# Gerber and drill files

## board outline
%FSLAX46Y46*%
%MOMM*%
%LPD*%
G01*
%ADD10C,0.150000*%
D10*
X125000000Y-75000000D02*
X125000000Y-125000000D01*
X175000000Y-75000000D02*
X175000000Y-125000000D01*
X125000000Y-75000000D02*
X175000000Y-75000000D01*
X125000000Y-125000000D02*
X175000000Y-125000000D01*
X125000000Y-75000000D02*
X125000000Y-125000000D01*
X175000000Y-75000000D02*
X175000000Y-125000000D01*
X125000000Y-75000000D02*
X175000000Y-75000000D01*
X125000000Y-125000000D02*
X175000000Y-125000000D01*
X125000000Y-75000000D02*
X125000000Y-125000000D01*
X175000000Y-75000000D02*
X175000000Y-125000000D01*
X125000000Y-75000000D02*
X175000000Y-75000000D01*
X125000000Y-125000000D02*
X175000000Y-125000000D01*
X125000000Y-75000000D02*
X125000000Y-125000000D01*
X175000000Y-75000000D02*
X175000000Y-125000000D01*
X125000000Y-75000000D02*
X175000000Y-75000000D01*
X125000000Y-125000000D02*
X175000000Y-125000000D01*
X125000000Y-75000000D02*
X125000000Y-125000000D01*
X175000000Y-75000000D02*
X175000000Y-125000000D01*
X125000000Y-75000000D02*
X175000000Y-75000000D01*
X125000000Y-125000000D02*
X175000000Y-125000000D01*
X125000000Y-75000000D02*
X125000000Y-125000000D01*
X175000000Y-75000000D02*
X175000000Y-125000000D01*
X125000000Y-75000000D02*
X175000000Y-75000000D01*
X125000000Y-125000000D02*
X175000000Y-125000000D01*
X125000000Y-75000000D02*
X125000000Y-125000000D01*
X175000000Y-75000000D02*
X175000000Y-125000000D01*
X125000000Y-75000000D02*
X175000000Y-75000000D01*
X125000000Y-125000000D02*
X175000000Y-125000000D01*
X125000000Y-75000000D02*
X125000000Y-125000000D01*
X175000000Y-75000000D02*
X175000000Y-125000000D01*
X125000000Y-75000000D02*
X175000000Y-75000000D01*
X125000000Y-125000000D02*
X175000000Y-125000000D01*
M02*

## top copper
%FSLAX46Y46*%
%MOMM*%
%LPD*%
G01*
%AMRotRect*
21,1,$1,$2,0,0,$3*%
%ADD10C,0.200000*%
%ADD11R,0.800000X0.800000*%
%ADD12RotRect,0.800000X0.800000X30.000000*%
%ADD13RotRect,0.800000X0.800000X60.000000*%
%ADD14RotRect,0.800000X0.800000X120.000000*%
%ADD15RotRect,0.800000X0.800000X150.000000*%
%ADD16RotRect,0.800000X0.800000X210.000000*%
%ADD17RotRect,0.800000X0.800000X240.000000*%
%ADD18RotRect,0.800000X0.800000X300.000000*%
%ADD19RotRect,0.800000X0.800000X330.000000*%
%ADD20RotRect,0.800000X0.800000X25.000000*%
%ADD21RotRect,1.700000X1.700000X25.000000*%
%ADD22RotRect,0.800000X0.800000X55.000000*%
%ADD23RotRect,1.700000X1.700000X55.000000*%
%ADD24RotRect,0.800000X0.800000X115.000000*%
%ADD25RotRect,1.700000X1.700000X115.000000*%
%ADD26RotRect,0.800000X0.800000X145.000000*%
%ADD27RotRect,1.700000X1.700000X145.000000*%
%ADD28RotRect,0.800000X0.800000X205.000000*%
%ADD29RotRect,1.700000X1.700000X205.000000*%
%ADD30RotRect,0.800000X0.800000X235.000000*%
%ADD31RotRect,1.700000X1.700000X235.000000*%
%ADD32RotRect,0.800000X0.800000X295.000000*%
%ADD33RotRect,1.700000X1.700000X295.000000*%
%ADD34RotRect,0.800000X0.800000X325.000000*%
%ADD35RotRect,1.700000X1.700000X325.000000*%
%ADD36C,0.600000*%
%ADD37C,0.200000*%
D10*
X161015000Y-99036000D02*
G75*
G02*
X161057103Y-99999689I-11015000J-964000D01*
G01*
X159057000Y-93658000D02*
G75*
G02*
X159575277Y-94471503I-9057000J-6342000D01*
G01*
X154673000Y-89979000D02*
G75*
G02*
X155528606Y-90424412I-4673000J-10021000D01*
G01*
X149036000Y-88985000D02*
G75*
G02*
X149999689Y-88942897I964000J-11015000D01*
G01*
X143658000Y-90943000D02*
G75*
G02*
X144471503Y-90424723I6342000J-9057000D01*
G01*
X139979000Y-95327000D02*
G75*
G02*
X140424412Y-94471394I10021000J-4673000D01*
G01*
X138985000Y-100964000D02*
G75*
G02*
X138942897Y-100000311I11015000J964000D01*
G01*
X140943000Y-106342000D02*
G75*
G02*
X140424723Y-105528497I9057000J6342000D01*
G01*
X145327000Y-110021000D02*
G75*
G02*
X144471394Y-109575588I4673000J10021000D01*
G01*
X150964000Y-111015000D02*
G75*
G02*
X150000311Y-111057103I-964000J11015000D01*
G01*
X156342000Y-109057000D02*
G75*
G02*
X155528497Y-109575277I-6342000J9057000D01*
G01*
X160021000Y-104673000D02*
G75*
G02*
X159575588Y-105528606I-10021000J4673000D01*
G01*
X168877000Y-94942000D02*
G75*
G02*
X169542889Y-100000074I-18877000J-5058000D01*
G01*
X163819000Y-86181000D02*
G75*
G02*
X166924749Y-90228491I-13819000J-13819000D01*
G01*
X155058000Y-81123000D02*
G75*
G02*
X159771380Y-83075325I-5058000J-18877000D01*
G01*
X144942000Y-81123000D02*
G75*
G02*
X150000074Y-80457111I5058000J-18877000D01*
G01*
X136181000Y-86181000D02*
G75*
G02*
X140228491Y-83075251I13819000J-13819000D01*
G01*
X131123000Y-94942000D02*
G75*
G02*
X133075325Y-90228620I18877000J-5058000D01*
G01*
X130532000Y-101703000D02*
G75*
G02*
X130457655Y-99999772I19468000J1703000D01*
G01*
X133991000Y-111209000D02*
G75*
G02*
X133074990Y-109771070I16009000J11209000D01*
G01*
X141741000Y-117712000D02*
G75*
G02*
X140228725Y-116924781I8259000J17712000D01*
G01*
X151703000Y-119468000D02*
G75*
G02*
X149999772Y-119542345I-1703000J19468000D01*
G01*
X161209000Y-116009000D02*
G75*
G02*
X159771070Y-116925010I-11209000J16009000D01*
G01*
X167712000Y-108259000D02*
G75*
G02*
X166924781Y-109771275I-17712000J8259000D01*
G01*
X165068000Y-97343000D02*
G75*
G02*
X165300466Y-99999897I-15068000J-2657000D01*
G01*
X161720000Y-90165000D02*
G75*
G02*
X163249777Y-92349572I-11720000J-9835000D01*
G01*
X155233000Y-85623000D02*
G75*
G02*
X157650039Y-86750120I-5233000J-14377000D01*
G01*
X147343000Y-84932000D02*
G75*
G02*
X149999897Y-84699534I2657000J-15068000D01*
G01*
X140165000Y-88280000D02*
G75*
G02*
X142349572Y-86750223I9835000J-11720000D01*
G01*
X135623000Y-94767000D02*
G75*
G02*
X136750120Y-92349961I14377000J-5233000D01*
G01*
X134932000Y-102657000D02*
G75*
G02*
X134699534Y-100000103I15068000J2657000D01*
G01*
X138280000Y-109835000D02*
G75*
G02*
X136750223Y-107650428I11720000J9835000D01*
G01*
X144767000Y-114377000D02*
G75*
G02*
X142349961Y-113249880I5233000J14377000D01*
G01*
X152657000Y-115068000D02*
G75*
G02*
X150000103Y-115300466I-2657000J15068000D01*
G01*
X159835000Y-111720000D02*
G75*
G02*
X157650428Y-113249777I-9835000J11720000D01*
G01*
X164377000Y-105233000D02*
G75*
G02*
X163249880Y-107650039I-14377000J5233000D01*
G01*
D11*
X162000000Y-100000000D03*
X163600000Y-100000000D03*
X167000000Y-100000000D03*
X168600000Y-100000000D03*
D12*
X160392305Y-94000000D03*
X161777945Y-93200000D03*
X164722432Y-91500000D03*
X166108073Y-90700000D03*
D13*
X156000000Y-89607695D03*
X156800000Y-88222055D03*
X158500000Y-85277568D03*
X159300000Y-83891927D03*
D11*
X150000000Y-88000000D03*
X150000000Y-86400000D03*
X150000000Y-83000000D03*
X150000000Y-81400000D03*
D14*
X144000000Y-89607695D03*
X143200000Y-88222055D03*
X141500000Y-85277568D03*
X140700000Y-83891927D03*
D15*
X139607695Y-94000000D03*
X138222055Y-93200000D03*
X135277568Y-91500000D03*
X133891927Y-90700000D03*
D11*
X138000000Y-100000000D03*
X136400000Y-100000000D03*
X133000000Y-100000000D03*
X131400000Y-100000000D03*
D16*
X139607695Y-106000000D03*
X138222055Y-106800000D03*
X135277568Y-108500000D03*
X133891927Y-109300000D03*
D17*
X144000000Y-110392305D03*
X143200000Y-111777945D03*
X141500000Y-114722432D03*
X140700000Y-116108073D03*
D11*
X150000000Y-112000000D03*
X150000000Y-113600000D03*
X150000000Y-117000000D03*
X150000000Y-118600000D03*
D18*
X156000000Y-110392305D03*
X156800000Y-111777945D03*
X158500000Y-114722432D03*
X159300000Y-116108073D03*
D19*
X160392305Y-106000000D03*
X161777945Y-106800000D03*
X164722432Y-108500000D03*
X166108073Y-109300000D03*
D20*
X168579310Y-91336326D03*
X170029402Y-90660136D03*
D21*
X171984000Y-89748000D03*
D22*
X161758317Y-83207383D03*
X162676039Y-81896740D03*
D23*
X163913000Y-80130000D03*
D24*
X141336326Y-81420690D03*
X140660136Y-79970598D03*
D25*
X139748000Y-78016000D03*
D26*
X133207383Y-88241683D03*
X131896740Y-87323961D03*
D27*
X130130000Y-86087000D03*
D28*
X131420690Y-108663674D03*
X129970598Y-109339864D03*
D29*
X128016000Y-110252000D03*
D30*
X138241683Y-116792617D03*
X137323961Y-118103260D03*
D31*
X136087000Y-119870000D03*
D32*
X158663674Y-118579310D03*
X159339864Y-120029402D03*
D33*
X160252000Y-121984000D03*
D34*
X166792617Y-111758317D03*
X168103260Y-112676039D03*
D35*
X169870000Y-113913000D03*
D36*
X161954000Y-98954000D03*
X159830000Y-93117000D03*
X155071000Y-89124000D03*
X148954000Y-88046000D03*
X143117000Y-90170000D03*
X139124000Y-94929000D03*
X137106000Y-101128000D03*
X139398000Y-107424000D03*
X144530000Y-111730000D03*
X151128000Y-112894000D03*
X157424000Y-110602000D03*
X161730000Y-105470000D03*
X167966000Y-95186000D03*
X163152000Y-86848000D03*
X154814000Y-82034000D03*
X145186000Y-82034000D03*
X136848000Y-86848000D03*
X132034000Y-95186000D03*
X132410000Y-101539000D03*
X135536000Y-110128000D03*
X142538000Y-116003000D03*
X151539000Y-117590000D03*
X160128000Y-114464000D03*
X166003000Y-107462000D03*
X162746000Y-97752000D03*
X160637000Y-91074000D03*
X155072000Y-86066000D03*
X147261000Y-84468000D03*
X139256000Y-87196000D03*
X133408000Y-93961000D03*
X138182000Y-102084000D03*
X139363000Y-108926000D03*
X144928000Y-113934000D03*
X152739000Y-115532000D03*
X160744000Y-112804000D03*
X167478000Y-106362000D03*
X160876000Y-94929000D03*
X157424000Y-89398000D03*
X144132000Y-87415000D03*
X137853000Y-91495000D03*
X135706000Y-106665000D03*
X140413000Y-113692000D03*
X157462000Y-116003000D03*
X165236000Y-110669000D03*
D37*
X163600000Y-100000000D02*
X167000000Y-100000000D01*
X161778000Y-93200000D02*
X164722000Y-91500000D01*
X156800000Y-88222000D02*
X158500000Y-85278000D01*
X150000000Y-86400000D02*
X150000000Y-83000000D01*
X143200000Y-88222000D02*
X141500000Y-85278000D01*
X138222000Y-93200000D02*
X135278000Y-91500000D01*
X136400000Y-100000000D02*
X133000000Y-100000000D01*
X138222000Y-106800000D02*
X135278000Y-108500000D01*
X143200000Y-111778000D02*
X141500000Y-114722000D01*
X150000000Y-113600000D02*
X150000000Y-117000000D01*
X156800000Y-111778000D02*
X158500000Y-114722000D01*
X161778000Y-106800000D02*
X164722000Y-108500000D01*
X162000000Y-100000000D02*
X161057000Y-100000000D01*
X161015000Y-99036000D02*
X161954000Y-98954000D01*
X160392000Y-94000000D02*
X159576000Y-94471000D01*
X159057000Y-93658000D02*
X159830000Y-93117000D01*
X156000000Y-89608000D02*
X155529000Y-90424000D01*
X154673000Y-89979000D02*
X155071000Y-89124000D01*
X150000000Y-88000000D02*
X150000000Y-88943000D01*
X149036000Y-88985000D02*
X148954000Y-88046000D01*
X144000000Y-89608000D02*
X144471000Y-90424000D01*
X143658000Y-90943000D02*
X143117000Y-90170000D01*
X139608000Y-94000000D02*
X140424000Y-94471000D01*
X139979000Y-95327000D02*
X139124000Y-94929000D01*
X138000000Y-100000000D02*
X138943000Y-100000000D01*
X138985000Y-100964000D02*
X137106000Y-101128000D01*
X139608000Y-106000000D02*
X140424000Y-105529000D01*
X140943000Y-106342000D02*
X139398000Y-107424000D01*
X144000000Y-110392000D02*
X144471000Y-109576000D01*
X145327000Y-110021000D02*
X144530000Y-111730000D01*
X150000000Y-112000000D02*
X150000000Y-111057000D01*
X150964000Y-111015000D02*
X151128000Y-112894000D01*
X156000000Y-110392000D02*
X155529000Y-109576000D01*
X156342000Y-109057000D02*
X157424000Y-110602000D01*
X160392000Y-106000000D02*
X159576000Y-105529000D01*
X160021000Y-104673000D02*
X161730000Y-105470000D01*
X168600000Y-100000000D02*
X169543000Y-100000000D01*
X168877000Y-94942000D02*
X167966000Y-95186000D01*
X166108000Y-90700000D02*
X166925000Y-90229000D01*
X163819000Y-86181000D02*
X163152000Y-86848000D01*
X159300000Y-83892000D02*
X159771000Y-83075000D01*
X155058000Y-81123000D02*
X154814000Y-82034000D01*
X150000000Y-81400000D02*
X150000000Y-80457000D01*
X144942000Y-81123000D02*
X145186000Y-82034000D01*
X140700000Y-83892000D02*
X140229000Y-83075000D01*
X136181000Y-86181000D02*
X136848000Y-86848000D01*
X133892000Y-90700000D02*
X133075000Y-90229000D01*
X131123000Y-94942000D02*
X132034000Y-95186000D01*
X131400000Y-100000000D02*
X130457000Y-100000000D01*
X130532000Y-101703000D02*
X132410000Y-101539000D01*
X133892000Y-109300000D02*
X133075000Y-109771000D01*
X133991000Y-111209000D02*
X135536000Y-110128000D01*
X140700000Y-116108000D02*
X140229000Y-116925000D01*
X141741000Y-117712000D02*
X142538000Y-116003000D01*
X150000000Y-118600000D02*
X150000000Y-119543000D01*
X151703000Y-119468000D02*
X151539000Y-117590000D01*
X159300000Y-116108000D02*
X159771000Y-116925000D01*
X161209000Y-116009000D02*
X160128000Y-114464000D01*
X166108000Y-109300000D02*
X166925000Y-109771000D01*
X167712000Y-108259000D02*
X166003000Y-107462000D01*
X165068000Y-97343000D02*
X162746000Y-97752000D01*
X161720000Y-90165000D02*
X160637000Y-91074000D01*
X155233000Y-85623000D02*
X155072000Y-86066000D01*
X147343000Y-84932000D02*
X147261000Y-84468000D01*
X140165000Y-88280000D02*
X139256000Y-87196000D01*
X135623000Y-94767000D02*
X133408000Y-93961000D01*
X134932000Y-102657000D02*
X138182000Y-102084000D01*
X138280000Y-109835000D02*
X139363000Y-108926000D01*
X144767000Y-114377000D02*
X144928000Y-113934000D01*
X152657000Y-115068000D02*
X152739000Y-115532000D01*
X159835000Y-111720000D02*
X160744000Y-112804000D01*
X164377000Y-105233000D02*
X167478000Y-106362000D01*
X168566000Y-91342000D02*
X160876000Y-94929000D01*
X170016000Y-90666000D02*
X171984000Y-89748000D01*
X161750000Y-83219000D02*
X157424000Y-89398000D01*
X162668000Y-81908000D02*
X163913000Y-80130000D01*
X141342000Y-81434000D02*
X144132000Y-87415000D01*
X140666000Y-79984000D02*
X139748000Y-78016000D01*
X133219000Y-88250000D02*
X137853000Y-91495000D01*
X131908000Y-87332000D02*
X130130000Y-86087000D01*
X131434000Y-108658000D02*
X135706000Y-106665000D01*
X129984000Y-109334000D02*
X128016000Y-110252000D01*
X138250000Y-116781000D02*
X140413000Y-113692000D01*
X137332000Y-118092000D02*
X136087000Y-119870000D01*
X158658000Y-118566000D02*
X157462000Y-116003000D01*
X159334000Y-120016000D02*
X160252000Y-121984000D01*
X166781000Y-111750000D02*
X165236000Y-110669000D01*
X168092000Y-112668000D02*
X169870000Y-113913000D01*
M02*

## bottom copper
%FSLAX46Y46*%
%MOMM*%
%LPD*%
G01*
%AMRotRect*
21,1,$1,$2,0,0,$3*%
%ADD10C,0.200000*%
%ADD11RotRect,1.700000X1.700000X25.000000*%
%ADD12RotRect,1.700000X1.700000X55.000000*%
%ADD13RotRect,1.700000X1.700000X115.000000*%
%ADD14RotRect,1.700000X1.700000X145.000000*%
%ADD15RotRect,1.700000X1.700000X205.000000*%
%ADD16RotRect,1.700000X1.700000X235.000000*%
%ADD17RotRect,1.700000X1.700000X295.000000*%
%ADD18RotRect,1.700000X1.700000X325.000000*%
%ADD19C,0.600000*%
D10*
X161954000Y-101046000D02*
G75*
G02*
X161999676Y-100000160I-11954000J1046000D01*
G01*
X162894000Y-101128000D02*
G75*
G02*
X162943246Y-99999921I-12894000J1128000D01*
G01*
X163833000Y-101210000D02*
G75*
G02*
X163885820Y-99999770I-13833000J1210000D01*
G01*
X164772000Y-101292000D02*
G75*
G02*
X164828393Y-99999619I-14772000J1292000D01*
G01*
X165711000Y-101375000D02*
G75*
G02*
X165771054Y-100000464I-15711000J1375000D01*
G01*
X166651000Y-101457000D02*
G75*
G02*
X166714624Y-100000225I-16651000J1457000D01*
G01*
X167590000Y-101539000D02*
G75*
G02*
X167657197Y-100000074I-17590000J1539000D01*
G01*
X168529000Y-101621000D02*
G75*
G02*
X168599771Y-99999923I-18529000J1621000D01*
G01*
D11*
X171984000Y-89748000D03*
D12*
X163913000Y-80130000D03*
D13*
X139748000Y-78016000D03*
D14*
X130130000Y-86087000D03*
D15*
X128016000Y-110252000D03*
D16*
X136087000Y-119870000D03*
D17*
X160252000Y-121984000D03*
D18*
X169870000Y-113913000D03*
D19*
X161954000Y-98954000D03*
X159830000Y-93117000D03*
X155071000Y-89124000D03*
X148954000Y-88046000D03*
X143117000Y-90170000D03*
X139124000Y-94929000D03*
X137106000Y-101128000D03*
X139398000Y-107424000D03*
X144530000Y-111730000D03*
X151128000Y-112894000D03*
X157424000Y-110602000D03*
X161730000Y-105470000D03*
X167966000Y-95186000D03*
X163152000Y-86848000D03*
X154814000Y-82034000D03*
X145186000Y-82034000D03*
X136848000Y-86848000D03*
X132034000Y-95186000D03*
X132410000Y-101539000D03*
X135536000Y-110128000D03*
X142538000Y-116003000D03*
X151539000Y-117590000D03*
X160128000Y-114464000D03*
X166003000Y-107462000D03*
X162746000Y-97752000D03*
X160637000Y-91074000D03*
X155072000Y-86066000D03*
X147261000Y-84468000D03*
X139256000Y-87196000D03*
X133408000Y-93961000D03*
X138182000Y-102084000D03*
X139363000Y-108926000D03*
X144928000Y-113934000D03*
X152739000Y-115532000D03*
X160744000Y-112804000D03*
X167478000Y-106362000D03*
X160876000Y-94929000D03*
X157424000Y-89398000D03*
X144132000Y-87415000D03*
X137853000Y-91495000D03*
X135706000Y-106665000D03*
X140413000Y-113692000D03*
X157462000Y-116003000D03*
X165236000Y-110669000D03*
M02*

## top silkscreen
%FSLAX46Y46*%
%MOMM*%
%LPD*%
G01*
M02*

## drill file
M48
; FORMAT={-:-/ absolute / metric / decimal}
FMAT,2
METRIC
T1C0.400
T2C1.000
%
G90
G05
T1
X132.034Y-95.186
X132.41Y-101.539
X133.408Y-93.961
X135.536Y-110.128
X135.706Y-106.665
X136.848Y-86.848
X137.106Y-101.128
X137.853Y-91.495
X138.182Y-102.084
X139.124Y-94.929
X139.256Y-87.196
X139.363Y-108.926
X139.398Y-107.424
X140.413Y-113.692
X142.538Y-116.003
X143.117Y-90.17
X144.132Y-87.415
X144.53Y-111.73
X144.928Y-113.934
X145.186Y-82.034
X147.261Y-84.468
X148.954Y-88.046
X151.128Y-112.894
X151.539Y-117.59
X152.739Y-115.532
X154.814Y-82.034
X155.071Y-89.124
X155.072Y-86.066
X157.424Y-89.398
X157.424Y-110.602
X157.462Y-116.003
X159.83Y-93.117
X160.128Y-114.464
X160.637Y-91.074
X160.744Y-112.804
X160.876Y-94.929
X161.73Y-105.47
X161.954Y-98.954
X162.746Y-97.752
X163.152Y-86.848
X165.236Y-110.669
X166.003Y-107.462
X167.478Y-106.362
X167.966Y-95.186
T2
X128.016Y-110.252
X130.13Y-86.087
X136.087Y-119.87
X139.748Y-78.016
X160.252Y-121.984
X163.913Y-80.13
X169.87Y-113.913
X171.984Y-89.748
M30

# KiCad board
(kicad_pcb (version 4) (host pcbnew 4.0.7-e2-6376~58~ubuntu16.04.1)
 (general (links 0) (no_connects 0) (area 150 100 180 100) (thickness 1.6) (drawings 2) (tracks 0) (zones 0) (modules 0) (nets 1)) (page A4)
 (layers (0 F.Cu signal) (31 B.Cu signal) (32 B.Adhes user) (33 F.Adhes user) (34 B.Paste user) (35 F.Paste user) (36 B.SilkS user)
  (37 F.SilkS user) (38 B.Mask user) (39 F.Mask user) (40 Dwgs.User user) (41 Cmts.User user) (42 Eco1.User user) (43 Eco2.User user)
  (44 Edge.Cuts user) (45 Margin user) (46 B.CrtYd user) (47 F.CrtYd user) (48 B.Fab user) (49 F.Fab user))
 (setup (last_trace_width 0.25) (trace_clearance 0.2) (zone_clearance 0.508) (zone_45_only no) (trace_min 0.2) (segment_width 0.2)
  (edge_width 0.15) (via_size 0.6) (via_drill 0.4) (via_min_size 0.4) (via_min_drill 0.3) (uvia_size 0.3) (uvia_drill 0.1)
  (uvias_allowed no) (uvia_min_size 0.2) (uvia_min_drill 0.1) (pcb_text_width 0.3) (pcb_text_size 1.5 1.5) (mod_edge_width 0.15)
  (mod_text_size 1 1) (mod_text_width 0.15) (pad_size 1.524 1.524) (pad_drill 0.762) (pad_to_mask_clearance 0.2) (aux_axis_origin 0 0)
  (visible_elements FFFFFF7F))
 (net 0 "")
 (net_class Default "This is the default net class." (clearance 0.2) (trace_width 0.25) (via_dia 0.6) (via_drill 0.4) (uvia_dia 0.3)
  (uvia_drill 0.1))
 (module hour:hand (layer F.Cu) (at 150 100 0.0)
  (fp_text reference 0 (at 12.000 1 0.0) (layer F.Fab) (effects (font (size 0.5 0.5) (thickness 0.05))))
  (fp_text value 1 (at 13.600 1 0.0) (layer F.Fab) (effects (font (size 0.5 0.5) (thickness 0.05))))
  (pad 1 smd rect (at 12.0 0 0.0) (size 0.8 0.8) (layers F.Cu F.Paste F.Mask))
  (pad 2 smd rect (at 13.6 0 0.0) (size 0.8 0.8) (layers F.Cu F.Paste F.Mask)))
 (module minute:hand (layer F.Cu) (at 150 100 0.0)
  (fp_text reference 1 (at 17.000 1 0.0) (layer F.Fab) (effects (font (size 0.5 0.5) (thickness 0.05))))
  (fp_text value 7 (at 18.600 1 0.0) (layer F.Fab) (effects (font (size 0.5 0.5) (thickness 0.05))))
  (pad 1 smd rect (at 17.0 0 0.0) (size 0.8 0.8) (layers F.Cu F.Paste F.Mask))
  (pad 2 smd rect (at 18.6 0 0.0) (size 0.8 0.8) (layers F.Cu F.Paste F.Mask)))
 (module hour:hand (layer F.Cu) (at 150 100 30.0)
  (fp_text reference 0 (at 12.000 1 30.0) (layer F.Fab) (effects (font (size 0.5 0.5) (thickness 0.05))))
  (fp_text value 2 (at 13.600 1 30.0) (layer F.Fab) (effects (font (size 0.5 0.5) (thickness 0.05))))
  (pad 1 smd rect (at 12.0 0 30.0) (size 0.8 0.8) (layers F.Cu F.Paste F.Mask))
  (pad 2 smd rect (at 13.6 0 30.0) (size 0.8 0.8) (layers F.Cu F.Paste F.Mask)))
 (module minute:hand (layer F.Cu) (at 150 100 30.0)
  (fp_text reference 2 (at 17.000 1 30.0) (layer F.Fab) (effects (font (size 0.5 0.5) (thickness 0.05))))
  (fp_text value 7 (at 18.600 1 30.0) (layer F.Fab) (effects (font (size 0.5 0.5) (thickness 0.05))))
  (pad 1 smd rect (at 17.0 0 30.0) (size 0.8 0.8) (layers F.Cu F.Paste F.Mask))
  (pad 2 smd rect (at 18.6 0 30.0) (size 0.8 0.8) (layers F.Cu F.Paste F.Mask)))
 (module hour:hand (layer F.Cu) (at 150 100 60.0)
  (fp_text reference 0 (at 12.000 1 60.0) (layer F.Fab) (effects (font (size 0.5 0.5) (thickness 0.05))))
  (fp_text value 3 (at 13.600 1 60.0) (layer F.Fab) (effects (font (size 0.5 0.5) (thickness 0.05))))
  (pad 1 smd rect (at 12.0 0 60.0) (size 0.8 0.8) (layers F.Cu F.Paste F.Mask))
  (pad 2 smd rect (at 13.6 0 60.0) (size 0.8 0.8) (layers F.Cu F.Paste F.Mask)))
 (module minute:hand (layer F.Cu) (at 150 100 60.0)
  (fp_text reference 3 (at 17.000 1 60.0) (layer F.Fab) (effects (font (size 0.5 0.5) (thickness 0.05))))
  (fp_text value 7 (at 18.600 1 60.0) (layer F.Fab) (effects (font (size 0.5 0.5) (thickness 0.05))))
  (pad 1 smd rect (at 17.0 0 60.0) (size 0.8 0.8) (layers F.Cu F.Paste F.Mask))
  (pad 2 smd rect (at 18.6 0 60.0) (size 0.8 0.8) (layers F.Cu F.Paste F.Mask)))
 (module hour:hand (layer F.Cu) (at 150 100 90.0)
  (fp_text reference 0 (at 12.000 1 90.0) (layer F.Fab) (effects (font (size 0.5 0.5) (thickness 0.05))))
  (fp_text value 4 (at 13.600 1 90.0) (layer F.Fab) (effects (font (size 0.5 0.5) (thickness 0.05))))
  (pad 1 smd rect (at 12.0 0 90.0) (size 0.8 0.8) (layers F.Cu F.Paste F.Mask))
  (pad 2 smd rect (at 13.6 0 90.0) (size 0.8 0.8) (layers F.Cu F.Paste F.Mask)))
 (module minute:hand (layer F.Cu) (at 150 100 90.0)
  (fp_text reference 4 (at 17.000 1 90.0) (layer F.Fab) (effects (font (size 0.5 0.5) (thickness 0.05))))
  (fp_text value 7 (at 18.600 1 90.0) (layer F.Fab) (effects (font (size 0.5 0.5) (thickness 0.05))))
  (pad 1 smd rect (at 17.0 0 90.0) (size 0.8 0.8) (layers F.Cu F.Paste F.Mask))
  (pad 2 smd rect (at 18.6 0 90.0) (size 0.8 0.8) (layers F.Cu F.Paste F.Mask)))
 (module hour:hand (layer F.Cu) (at 150 100 120.0)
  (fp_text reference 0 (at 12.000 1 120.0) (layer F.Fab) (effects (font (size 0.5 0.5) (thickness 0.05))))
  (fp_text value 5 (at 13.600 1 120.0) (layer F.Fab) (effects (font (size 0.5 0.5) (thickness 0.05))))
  (pad 1 smd rect (at 12.0 0 120.0) (size 0.8 0.8) (layers F.Cu F.Paste F.Mask))
  (pad 2 smd rect (at 13.6 0 120.0) (size 0.8 0.8) (layers F.Cu F.Paste F.Mask)))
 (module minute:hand (layer F.Cu) (at 150 100 120.0)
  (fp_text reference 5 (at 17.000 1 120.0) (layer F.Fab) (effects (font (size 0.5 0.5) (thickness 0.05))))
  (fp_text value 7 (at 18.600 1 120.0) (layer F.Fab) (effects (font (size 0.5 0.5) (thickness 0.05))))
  (pad 1 smd rect (at 17.0 0 120.0) (size 0.8 0.8) (layers F.Cu F.Paste F.Mask))
  (pad 2 smd rect (at 18.6 0 120.0) (size 0.8 0.8) (layers F.Cu F.Paste F.Mask)))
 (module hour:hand (layer F.Cu) (at 150 100 150.0)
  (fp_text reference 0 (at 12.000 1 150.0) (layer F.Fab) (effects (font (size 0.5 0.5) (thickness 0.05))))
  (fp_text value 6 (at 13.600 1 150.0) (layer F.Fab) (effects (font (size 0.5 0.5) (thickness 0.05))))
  (pad 1 smd rect (at 12.0 0 150.0) (size 0.8 0.8) (layers F.Cu F.Paste F.Mask))
  (pad 2 smd rect (at 13.6 0 150.0) (size 0.8 0.8) (layers F.Cu F.Paste F.Mask)))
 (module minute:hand (layer F.Cu) (at 150 100 150.0)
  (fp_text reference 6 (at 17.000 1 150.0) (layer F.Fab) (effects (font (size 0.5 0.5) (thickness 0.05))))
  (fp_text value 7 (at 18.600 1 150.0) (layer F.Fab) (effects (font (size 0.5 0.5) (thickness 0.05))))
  (pad 1 smd rect (at 17.0 0 150.0) (size 0.8 0.8) (layers F.Cu F.Paste F.Mask))
  (pad 2 smd rect (at 18.6 0 150.0) (size 0.8 0.8) (layers F.Cu F.Paste F.Mask)))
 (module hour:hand (layer F.Cu) (at 150 100 180.0)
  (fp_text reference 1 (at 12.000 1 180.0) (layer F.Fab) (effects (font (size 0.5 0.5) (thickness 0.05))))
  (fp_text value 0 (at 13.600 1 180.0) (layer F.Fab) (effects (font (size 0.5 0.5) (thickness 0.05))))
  (pad 1 smd rect (at 12.0 0 180.0) (size 0.8 0.8) (layers F.Cu F.Paste F.Mask))
  (pad 2 smd rect (at 13.6 0 180.0) (size 0.8 0.8) (layers F.Cu F.Paste F.Mask)))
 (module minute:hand (layer F.Cu) (at 150 100 180.0)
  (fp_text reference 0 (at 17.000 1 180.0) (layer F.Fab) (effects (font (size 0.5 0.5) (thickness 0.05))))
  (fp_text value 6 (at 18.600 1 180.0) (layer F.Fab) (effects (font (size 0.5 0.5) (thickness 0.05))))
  (pad 1 smd rect (at 17.0 0 180.0) (size 0.8 0.8) (layers F.Cu F.Paste F.Mask))
  (pad 2 smd rect (at 18.6 0 180.0) (size 0.8 0.8) (layers F.Cu F.Paste F.Mask)))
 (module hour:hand (layer F.Cu) (at 150 100 210.0)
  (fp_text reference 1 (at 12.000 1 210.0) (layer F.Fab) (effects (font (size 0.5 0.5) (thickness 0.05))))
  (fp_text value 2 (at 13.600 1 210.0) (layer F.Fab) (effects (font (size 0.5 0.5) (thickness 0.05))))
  (pad 1 smd rect (at 12.0 0 210.0) (size 0.8 0.8) (layers F.Cu F.Paste F.Mask))
  (pad 2 smd rect (at 13.6 0 210.0) (size 0.8 0.8) (layers F.Cu F.Paste F.Mask)))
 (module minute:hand (layer F.Cu) (at 150 100 210.0)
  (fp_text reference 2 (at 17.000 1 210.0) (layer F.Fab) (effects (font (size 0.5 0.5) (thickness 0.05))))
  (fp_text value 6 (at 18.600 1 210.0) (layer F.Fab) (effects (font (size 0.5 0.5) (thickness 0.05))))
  (pad 1 smd rect (at 17.0 0 210.0) (size 0.8 0.8) (layers F.Cu F.Paste F.Mask))
  (pad 2 smd rect (at 18.6 0 210.0) (size 0.8 0.8) (layers F.Cu F.Paste F.Mask)))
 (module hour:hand (layer F.Cu) (at 150 100 240.0)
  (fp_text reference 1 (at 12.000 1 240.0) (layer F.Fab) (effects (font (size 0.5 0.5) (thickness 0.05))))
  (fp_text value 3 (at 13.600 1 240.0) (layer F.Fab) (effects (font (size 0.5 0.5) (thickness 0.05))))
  (pad 1 smd rect (at 12.0 0 240.0) (size 0.8 0.8) (layers F.Cu F.Paste F.Mask))
  (pad 2 smd rect (at 13.6 0 240.0) (size 0.8 0.8) (layers F.Cu F.Paste F.Mask)))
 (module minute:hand (layer F.Cu) (at 150 100 240.0)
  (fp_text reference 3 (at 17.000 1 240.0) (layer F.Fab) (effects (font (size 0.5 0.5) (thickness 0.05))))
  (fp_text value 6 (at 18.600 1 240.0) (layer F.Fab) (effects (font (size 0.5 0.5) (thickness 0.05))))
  (pad 1 smd rect (at 17.0 0 240.0) (size 0.8 0.8) (layers F.Cu F.Paste F.Mask))
  (pad 2 smd rect (at 18.6 0 240.0) (size 0.8 0.8) (layers F.Cu F.Paste F.Mask)))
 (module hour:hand (layer F.Cu) (at 150 100 270.0)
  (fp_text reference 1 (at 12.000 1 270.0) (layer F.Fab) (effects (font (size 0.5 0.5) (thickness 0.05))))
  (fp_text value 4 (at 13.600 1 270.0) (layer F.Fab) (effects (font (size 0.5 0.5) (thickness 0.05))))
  (pad 1 smd rect (at 12.0 0 270.0) (size 0.8 0.8) (layers F.Cu F.Paste F.Mask))
  (pad 2 smd rect (at 13.6 0 270.0) (size 0.8 0.8) (layers F.Cu F.Paste F.Mask)))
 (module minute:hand (layer F.Cu) (at 150 100 270.0)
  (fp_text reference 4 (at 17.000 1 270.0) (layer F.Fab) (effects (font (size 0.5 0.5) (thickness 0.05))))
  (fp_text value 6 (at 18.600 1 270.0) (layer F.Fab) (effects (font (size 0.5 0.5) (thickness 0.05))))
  (pad 1 smd rect (at 17.0 0 270.0) (size 0.8 0.8) (layers F.Cu F.Paste F.Mask))
  (pad 2 smd rect (at 18.6 0 270.0) (size 0.8 0.8) (layers F.Cu F.Paste F.Mask)))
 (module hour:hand (layer F.Cu) (at 150 100 300.0)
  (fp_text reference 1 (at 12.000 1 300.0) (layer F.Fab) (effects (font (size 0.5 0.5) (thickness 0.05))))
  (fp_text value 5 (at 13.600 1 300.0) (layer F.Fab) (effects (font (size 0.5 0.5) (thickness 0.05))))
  (pad 1 smd rect (at 12.0 0 300.0) (size 0.8 0.8) (layers F.Cu F.Paste F.Mask))
  (pad 2 smd rect (at 13.6 0 300.0) (size 0.8 0.8) (layers F.Cu F.Paste F.Mask)))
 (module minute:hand (layer F.Cu) (at 150 100 300.0)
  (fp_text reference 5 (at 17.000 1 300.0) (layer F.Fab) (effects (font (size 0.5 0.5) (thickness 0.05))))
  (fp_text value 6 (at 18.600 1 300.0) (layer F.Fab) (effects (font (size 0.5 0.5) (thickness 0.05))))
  (pad 1 smd rect (at 17.0 0 300.0) (size 0.8 0.8) (layers F.Cu F.Paste F.Mask))
  (pad 2 smd rect (at 18.6 0 300.0) (size 0.8 0.8) (layers F.Cu F.Paste F.Mask)))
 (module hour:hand (layer F.Cu) (at 150 100 330.0)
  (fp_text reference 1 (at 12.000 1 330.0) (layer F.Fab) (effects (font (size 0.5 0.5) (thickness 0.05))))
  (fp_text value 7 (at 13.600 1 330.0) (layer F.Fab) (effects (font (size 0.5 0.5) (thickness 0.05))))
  (pad 1 smd rect (at 12.0 0 330.0) (size 0.8 0.8) (layers F.Cu F.Paste F.Mask))
  (pad 2 smd rect (at 13.6 0 330.0) (size 0.8 0.8) (layers F.Cu F.Paste F.Mask)))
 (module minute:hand (layer F.Cu) (at 150 100 330.0)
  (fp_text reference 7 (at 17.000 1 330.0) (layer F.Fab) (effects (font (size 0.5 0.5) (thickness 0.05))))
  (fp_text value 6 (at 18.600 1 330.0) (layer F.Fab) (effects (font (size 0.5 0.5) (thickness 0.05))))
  (pad 1 smd rect (at 17.0 0 330.0) (size 0.8 0.8) (layers F.Cu F.Paste F.Mask))
  (pad 2 smd rect (at 18.6 0 330.0) (size 0.8 0.8) (layers F.Cu F.Paste F.Mask)))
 (segment (start 163.600 100.000) (end 167.000 100.000) (width 0.2) (layer F.Cu) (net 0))
 (segment (start 161.778 93.200) (end 164.722 91.500) (width 0.2) (layer F.Cu) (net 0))
 (segment (start 156.800 88.222) (end 158.500 85.278) (width 0.2) (layer F.Cu) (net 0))
 (segment (start 150.000 86.400) (end 150.000 83.000) (width 0.2) (layer F.Cu) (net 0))
 (segment (start 143.200 88.222) (end 141.500 85.278) (width 0.2) (layer F.Cu) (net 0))
 (segment (start 138.222 93.200) (end 135.278 91.500) (width 0.2) (layer F.Cu) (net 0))
 (segment (start 136.400 100.000) (end 133.000 100.000) (width 0.2) (layer F.Cu) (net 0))
 (segment (start 138.222 106.800) (end 135.278 108.500) (width 0.2) (layer F.Cu) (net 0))
 (segment (start 143.200 111.778) (end 141.500 114.722) (width 0.2) (layer F.Cu) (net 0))
 (segment (start 150.000 113.600) (end 150.000 117.000) (width 0.2) (layer F.Cu) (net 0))
 (segment (start 156.800 111.778) (end 158.500 114.722) (width 0.2) (layer F.Cu) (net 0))
 (segment (start 161.778 106.800) (end 164.722 108.500) (width 0.2) (layer F.Cu) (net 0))
 (gr_arc (start 150 100) (end 161.954 101.046) (angle 355.000) (layer B.Cu) (width 0.2))
 (gr_arc (start 150 100) (end 162.894 101.128) (angle 355.000) (layer B.Cu) (width 0.2))
 (gr_arc (start 150 100) (end 163.833 101.210) (angle 355.000) (layer B.Cu) (width 0.2))
 (gr_arc (start 150 100) (end 164.772 101.292) (angle 355.000) (layer B.Cu) (width 0.2))
 (gr_arc (start 150 100) (end 165.711 101.375) (angle 355.000) (layer B.Cu) (width 0.2))
 (gr_arc (start 150 100) (end 166.651 101.457) (angle 355.000) (layer B.Cu) (width 0.2))
 (gr_arc (start 150 100) (end 167.590 101.539) (angle 355.000) (layer B.Cu) (width 0.2))
 (gr_arc (start 150 100) (end 168.529 101.621) (angle 355.000) (layer B.Cu) (width 0.2))
 (segment (start 162.000 100.000) (end 161.057 100.000) (width 0.2) (layer F.Cu) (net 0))
 (gr_arc (start 150 100) (end 161.015 99.036) (angle 5.000) (layer F.Cu) (width 0.2))
 (segment (start 161.015 99.036) (end 161.954 98.954) (width 0.2) (layer F.Cu) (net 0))
 (via (at 161.954 98.954) (size 0.6) (drill 0.4) (layers F.Cu B.Cu) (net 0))
 (segment (start 160.392 94.000) (end 159.576 94.471) (width 0.2) (layer F.Cu) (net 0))
 (gr_arc (start 150 100) (end 159.057 93.658) (angle 5.000) (layer F.Cu) (width 0.2))
 (segment (start 159.057 93.658) (end 159.830 93.117) (width 0.2) (layer F.Cu) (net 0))
 (via (at 159.830 93.117) (size 0.6) (drill 0.4) (layers F.Cu B.Cu) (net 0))
 (segment (start 156.000 89.608) (end 155.529 90.424) (width 0.2) (layer F.Cu) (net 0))
 (gr_arc (start 150 100) (end 154.673 89.979) (angle 5.000) (layer F.Cu) (width 0.2))
 (segment (start 154.673 89.979) (end 155.071 89.124) (width 0.2) (layer F.Cu) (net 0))
 (via (at 155.071 89.124) (size 0.6) (drill 0.4) (layers F.Cu B.Cu) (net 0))
 (segment (start 150.000 88.000) (end 150.000 88.943) (width 0.2) (layer F.Cu) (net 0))
 (gr_arc (start 150 100) (end 149.036 88.985) (angle 5.000) (layer F.Cu) (width 0.2))
 (segment (start 149.036 88.985) (end 148.954 88.046) (width 0.2) (layer F.Cu) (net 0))
 (via (at 148.954 88.046) (size 0.6) (drill 0.4) (layers F.Cu B.Cu) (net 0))
 (segment (start 144.000 89.608) (end 144.471 90.424) (width 0.2) (layer F.Cu) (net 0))
 (gr_arc (start 150 100) (end 143.658 90.943) (angle 5.000) (layer F.Cu) (width 0.2))
 (segment (start 143.658 90.943) (end 143.117 90.170) (width 0.2) (layer F.Cu) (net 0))
 (via (at 143.117 90.170) (size 0.6) (drill 0.4) (layers F.Cu B.Cu) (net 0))
 (segment (start 139.608 94.000) (end 140.424 94.471) (width 0.2) (layer F.Cu) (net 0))
 (gr_arc (start 150 100) (end 139.979 95.327) (angle 5.000) (layer F.Cu) (width 0.2))
 (segment (start 139.979 95.327) (end 139.124 94.929) (width 0.2) (layer F.Cu) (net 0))
 (via (at 139.124 94.929) (size 0.6) (drill 0.4) (layers F.Cu B.Cu) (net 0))
 (segment (start 138.000 100.000) (end 138.943 100.000) (width 0.2) (layer F.Cu) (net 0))
 (gr_arc (start 150 100) (end 138.985 100.964) (angle 5.000) (layer F.Cu) (width 0.2))
 (segment (start 138.985 100.964) (end 137.106 101.128) (width 0.2) (layer F.Cu) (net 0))
 (via (at 137.106 101.128) (size 0.6) (drill 0.4) (layers F.Cu B.Cu) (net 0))
 (segment (start 139.608 106.000) (end 140.424 105.529) (width 0.2) (layer F.Cu) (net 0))
 (gr_arc (start 150 100) (end 140.943 106.342) (angle 5.000) (layer F.Cu) (width 0.2))
 (segment (start 140.943 106.342) (end 139.398 107.424) (width 0.2) (layer F.Cu) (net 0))
 (via (at 139.398 107.424) (size 0.6) (drill 0.4) (layers F.Cu B.Cu) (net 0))
 (segment (start 144.000 110.392) (end 144.471 109.576) (width 0.2) (layer F.Cu) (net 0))
 (gr_arc (start 150 100) (end 145.327 110.021) (angle 5.000) (layer F.Cu) (width 0.2))
 (segment (start 145.327 110.021) (end 144.530 111.730) (width 0.2) (layer F.Cu) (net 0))
 (via (at 144.530 111.730) (size 0.6) (drill 0.4) (layers F.Cu B.Cu) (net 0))
 (segment (start 150.000 112.000) (end 150.000 111.057) (width 0.2) (layer F.Cu) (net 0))
 (gr_arc (start 150 100) (end 150.964 111.015) (angle 5.000) (layer F.Cu) (width 0.2))
 (segment (start 150.964 111.015) (end 151.128 112.894) (width 0.2) (layer F.Cu) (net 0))
 (via (at 151.128 112.894) (size 0.6) (drill 0.4) (layers F.Cu B.Cu) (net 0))
 (segment (start 156.000 110.392) (end 155.529 109.576) (width 0.2) (layer F.Cu) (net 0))
 (gr_arc (start 150 100) (end 156.342 109.057) (angle 5.000) (layer F.Cu) (width 0.2))
 (segment (start 156.342 109.057) (end 157.424 110.602) (width 0.2) (layer F.Cu) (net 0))
 (via (at 157.424 110.602) (size 0.6) (drill 0.4) (layers F.Cu B.Cu) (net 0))
 (segment (start 160.392 106.000) (end 159.576 105.529) (width 0.2) (layer F.Cu) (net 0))
 (gr_arc (start 150 100) (end 160.021 104.673) (angle 5.000) (layer F.Cu) (width 0.2))
 (segment (start 160.021 104.673) (end 161.730 105.470) (width 0.2) (layer F.Cu) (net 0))
 (via (at 161.730 105.470) (size 0.6) (drill 0.4) (layers F.Cu B.Cu) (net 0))
 (segment (start 168.600 100.000) (end 169.543 100.000) (width 0.2) (layer F.Cu) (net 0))
 (gr_arc (start 150 100) (end 168.877 94.942) (angle 15.000) (layer F.Cu) (width 0.2))
 (segment (start 168.877 94.942) (end 167.966 95.186) (width 0.2) (layer F.Cu) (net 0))
 (via (at 167.966 95.186) (size 0.6) (drill 0.4) (layers F.Cu B.Cu) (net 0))
 (segment (start 166.108 90.700) (end 166.925 90.229) (width 0.2) (layer F.Cu) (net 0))
 (gr_arc (start 150 100) (end 163.819 86.181) (angle 15.000) (layer F.Cu) (width 0.2))
 (segment (start 163.819 86.181) (end 163.152 86.848) (width 0.2) (layer F.Cu) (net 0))
 (via (at 163.152 86.848) (size 0.6) (drill 0.4) (layers F.Cu B.Cu) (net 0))
 (segment (start 159.300 83.892) (end 159.771 83.075) (width 0.2) (layer F.Cu) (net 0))
 (gr_arc (start 150 100) (end 155.058 81.123) (angle 15.000) (layer F.Cu) (width 0.2))
 (segment (start 155.058 81.123) (end 154.814 82.034) (width 0.2) (layer F.Cu) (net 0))
 (via (at 154.814 82.034) (size 0.6) (drill 0.4) (layers F.Cu B.Cu) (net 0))
 (segment (start 150.000 81.400) (end 150.000 80.457) (width 0.2) (layer F.Cu) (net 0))
 (gr_arc (start 150 100) (end 144.942 81.123) (angle 15.000) (layer F.Cu) (width 0.2))
 (segment (start 144.942 81.123) (end 145.186 82.034) (width 0.2) (layer F.Cu) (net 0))
 (via (at 145.186 82.034) (size 0.6) (drill 0.4) (layers F.Cu B.Cu) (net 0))
 (segment (start 140.700 83.892) (end 140.229 83.075) (width 0.2) (layer F.Cu) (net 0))
 (gr_arc (start 150 100) (end 136.181 86.181) (angle 15.000) (layer F.Cu) (width 0.2))
 (segment (start 136.181 86.181) (end 136.848 86.848) (width 0.2) (layer F.Cu) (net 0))
 (via (at 136.848 86.848) (size 0.6) (drill 0.4) (layers F.Cu B.Cu) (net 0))
 (segment (start 133.892 90.700) (end 133.075 90.229) (width 0.2) (layer F.Cu) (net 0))
 (gr_arc (start 150 100) (end 131.123 94.942) (angle 15.000) (layer F.Cu) (width 0.2))
 (segment (start 131.123 94.942) (end 132.034 95.186) (width 0.2) (layer F.Cu) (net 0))
 (via (at 132.034 95.186) (size 0.6) (drill 0.4) (layers F.Cu B.Cu) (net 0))
 (segment (start 131.400 100.000) (end 130.457 100.000) (width 0.2) (layer F.Cu) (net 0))
 (gr_arc (start 150 100) (end 130.532 101.703) (angle 5.000) (layer F.Cu) (width 0.2))
 (segment (start 130.532 101.703) (end 132.410 101.539) (width 0.2) (layer F.Cu) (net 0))
 (via (at 132.410 101.539) (size 0.6) (drill 0.4) (layers F.Cu B.Cu) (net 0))
 (segment (start 133.892 109.300) (end 133.075 109.771) (width 0.2) (layer F.Cu) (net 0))
 (gr_arc (start 150 100) (end 133.991 111.209) (angle 5.000) (layer F.Cu) (width 0.2))
 (segment (start 133.991 111.209) (end 135.536 110.128) (width 0.2) (layer F.Cu) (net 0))
 (via (at 135.536 110.128) (size 0.6) (drill 0.4) (layers F.Cu B.Cu) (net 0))
 (segment (start 140.700 116.108) (end 140.229 116.925) (width 0.2) (layer F.Cu) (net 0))
 (gr_arc (start 150 100) (end 141.741 117.712) (angle 5.000) (layer F.Cu) (width 0.2))
 (segment (start 141.741 117.712) (end 142.538 116.003) (width 0.2) (layer F.Cu) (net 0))
 (via (at 142.538 116.003) (size 0.6) (drill 0.4) (layers F.Cu B.Cu) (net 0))
 (segment (start 150.000 118.600) (end 150.000 119.543) (width 0.2) (layer F.Cu) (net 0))
 (gr_arc (start 150 100) (end 151.703 119.468) (angle 5.000) (layer F.Cu) (width 0.2))
 (segment (start 151.703 119.468) (end 151.539 117.590) (width 0.2) (layer F.Cu) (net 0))
 (via (at 151.539 117.590) (size 0.6) (drill 0.4) (layers F.Cu B.Cu) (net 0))
 (segment (start 159.300 116.108) (end 159.771 116.925) (width 0.2) (layer F.Cu) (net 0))
 (gr_arc (start 150 100) (end 161.209 116.009) (angle 5.000) (layer F.Cu) (width 0.2))
 (segment (start 161.209 116.009) (end 160.128 114.464) (width 0.2) (layer F.Cu) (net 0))
 (via (at 160.128 114.464) (size 0.6) (drill 0.4) (layers F.Cu B.Cu) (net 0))
 (segment (start 166.108 109.300) (end 166.925 109.771) (width 0.2) (layer F.Cu) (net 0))
 (gr_arc (start 150 100) (end 167.712 108.259) (angle 5.000) (layer F.Cu) (width 0.2))
 (segment (start 167.712 108.259) (end 166.003 107.462) (width 0.2) (layer F.Cu) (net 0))
 (via (at 166.003 107.462) (size 0.6) (drill 0.4) (layers F.Cu B.Cu) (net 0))
 (gr_arc (start 150 100) (end 165.068 97.343) (angle 10.000) (layer F.Cu) (width 0.2))
 (segment (start 165.068 97.343) (end 162.746 97.752) (width 0.2) (layer F.Cu) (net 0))
 (via (at 162.746 97.752) (size 0.6) (drill 0.4) (layers F.Cu B.Cu) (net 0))
 (gr_arc (start 150 100) (end 161.720 90.165) (angle 10.000) (layer F.Cu) (width 0.2))
 (segment (start 161.720 90.165) (end 160.637 91.074) (width 0.2) (layer F.Cu) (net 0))
 (via (at 160.637 91.074) (size 0.6) (drill 0.4) (layers F.Cu B.Cu) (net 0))
 (gr_arc (start 150 100) (end 155.233 85.623) (angle 10.000) (layer F.Cu) (width 0.2))
 (segment (start 155.233 85.623) (end 155.072 86.066) (width 0.2) (layer F.Cu) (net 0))
 (via (at 155.072 86.066) (size 0.6) (drill 0.4) (layers F.Cu B.Cu) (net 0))
 (gr_arc (start 150 100) (end 147.343 84.932) (angle 10.000) (layer F.Cu) (width 0.2))
 (segment (start 147.343 84.932) (end 147.261 84.468) (width 0.2) (layer F.Cu) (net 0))
 (via (at 147.261 84.468) (size 0.6) (drill 0.4) (layers F.Cu B.Cu) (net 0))
 (gr_arc (start 150 100) (end 140.165 88.280) (angle 10.000) (layer F.Cu) (width 0.2))
 (segment (start 140.165 88.280) (end 139.256 87.196) (width 0.2) (layer F.Cu) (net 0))
 (via (at 139.256 87.196) (size 0.6) (drill 0.4) (layers F.Cu B.Cu) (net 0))
 (gr_arc (start 150 100) (end 135.623 94.767) (angle 10.000) (layer F.Cu) (width 0.2))
 (segment (start 135.623 94.767) (end 133.408 93.961) (width 0.2) (layer F.Cu) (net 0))
 (via (at 133.408 93.961) (size 0.6) (drill 0.4) (layers F.Cu B.Cu) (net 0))
 (gr_arc (start 150 100) (end 134.932 102.657) (angle 10.000) (layer F.Cu) (width 0.2))
 (segment (start 134.932 102.657) (end 138.182 102.084) (width 0.2) (layer F.Cu) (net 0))
 (via (at 138.182 102.084) (size 0.6) (drill 0.4) (layers F.Cu B.Cu) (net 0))
 (gr_arc (start 150 100) (end 138.280 109.835) (angle 10.000) (layer F.Cu) (width 0.2))
 (segment (start 138.280 109.835) (end 139.363 108.926) (width 0.2) (layer F.Cu) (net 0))
 (via (at 139.363 108.926) (size 0.6) (drill 0.4) (layers F.Cu B.Cu) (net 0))
 (gr_arc (start 150 100) (end 144.767 114.377) (angle 10.000) (layer F.Cu) (width 0.2))
 (segment (start 144.767 114.377) (end 144.928 113.934) (width 0.2) (layer F.Cu) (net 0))
 (via (at 144.928 113.934) (size 0.6) (drill 0.4) (layers F.Cu B.Cu) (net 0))
 (gr_arc (start 150 100) (end 152.657 115.068) (angle 10.000) (layer F.Cu) (width 0.2))
 (segment (start 152.657 115.068) (end 152.739 115.532) (width 0.2) (layer F.Cu) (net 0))
 (via (at 152.739 115.532) (size 0.6) (drill 0.4) (layers F.Cu B.Cu) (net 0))
 (gr_arc (start 150 100) (end 159.835 111.720) (angle 10.000) (layer F.Cu) (width 0.2))
 (segment (start 159.835 111.720) (end 160.744 112.804) (width 0.2) (layer F.Cu) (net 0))
 (via (at 160.744 112.804) (size 0.6) (drill 0.4) (layers F.Cu B.Cu) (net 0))
 (gr_arc (start 150 100) (end 164.377 105.233) (angle 10.000) (layer F.Cu) (width 0.2))
 (segment (start 164.377 105.233) (end 167.478 106.362) (width 0.2) (layer F.Cu) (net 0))
 (via (at 167.478 106.362) (size 0.6) (drill 0.4) (layers F.Cu B.Cu) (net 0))
 (segment (start 168.566 91.342) (end 160.876 94.929) (width 0.2) (layer F.Cu) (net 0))
 (via (at 160.876 94.929) (size 0.6) (drill 0.4) (layers F.Cu B.Cu) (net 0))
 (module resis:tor (layer F.Cu) (at 150 100 25.0)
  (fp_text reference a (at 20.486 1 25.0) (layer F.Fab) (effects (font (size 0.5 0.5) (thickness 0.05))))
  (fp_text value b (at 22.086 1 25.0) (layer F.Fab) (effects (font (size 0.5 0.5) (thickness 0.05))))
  (pad 1 smd rect (at 20.5 0 25.0) (size 0.8 0.8) (layers F.Cu F.Paste F.Mask))
  (pad 2 smd rect (at 22.1 0 25.0) (size 0.8 0.8) (layers F.Cu F.Paste F.Mask)))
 (segment (start 170.016 90.666) (end 171.984 89.748) (width 0.2) (layer F.Cu) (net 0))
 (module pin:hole (layer F.Cu) (at 171.984 89.748)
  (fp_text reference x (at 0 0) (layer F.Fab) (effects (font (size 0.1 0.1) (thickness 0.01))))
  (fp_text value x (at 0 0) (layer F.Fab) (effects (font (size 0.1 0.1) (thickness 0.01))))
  (pad 0 thru_hole rect (at 0 0 25.0) (size 1.7 1.7) (drill 1) (layers *.Cu *.Mask)))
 (gr_line (start 125.000 75.000) (end 125.000 125.000) (angle 90) (layer Edge.Cuts) (width 0.15))
 (gr_line (start 175.000 75.000) (end 175.000 125.000) (angle 90) (layer Edge.Cuts) (width 0.15))
 (gr_line (start 125.000 75.000) (end 175.000 75.000) (angle 0) (layer Edge.Cuts) (width 0.15))
 (gr_line (start 125.000 125.000) (end 175.000 125.000) (angle 0) (layer Edge.Cuts) (width 0.15))
 (segment (start 161.750 83.219) (end 157.424 89.398) (width 0.2) (layer F.Cu) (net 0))
 (via (at 157.424 89.398) (size 0.6) (drill 0.4) (layers F.Cu B.Cu) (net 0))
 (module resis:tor (layer F.Cu) (at 150 100 55.0)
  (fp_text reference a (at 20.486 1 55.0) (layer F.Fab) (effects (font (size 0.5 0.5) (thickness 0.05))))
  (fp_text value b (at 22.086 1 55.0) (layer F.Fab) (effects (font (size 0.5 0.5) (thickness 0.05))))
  (pad 1 smd rect (at 20.5 0 55.0) (size 0.8 0.8) (layers F.Cu F.Paste F.Mask))
  (pad 2 smd rect (at 22.1 0 55.0) (size 0.8 0.8) (layers F.Cu F.Paste F.Mask)))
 (segment (start 162.668 81.908) (end 163.913 80.130) (width 0.2) (layer F.Cu) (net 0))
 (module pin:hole (layer F.Cu) (at 163.913 80.130)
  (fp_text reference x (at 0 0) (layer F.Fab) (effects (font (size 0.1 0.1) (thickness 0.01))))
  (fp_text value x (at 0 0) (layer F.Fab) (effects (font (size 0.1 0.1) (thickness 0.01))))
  (pad 1 thru_hole rect (at 0 0 55.0) (size 1.7 1.7) (drill 1) (layers *.Cu *.Mask)))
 (gr_line (start 125.000 75.000) (end 125.000 125.000) (angle 90) (layer Edge.Cuts) (width 0.15))
 (gr_line (start 175.000 75.000) (end 175.000 125.000) (angle 90) (layer Edge.Cuts) (width 0.15))
 (gr_line (start 125.000 75.000) (end 175.000 75.000) (angle 0) (layer Edge.Cuts) (width 0.15))
 (gr_line (start 125.000 125.000) (end 175.000 125.000) (angle 0) (layer Edge.Cuts) (width 0.15))
 (segment (start 141.342 81.434) (end 144.132 87.415) (width 0.2) (layer F.Cu) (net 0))
 (via (at 144.132 87.415) (size 0.6) (drill 0.4) (layers F.Cu B.Cu) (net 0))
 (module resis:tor (layer F.Cu) (at 150 100 115.0)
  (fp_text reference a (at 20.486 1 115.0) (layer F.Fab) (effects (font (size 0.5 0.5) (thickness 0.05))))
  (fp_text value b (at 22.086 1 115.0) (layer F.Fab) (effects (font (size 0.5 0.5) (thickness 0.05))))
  (pad 1 smd rect (at 20.5 0 115.0) (size 0.8 0.8) (layers F.Cu F.Paste F.Mask))
  (pad 2 smd rect (at 22.1 0 115.0) (size 0.8 0.8) (layers F.Cu F.Paste F.Mask)))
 (segment (start 140.666 79.984) (end 139.748 78.016) (width 0.2) (layer F.Cu) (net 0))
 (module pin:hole (layer F.Cu) (at 139.748 78.016)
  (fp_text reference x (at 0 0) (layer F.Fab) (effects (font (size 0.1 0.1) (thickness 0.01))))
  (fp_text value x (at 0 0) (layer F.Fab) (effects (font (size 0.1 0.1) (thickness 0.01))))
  (pad 2 thru_hole rect (at 0 0 115.0) (size 1.7 1.7) (drill 1) (layers *.Cu *.Mask)))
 (gr_line (start 125.000 75.000) (end 125.000 125.000) (angle 90) (layer Edge.Cuts) (width 0.15))
 (gr_line (start 175.000 75.000) (end 175.000 125.000) (angle 90) (layer Edge.Cuts) (width 0.15))
 (gr_line (start 125.000 75.000) (end 175.000 75.000) (angle 0) (layer Edge.Cuts) (width 0.15))
 (gr_line (start 125.000 125.000) (end 175.000 125.000) (angle 0) (layer Edge.Cuts) (width 0.15))
 (segment (start 133.219 88.250) (end 137.853 91.495) (width 0.2) (layer F.Cu) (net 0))
 (via (at 137.853 91.495) (size 0.6) (drill 0.4) (layers F.Cu B.Cu) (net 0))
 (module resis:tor (layer F.Cu) (at 150 100 145.0)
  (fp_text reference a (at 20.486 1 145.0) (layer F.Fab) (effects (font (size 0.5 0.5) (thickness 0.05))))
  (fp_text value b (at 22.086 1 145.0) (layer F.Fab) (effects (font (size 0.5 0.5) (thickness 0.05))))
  (pad 1 smd rect (at 20.5 0 145.0) (size 0.8 0.8) (layers F.Cu F.Paste F.Mask))
  (pad 2 smd rect (at 22.1 0 145.0) (size 0.8 0.8) (layers F.Cu F.Paste F.Mask)))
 (segment (start 131.908 87.332) (end 130.130 86.087) (width 0.2) (layer F.Cu) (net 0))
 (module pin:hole (layer F.Cu) (at 130.130 86.087)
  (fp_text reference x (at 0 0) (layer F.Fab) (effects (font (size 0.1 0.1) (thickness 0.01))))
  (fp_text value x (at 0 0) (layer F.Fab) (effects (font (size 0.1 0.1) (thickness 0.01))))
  (pad 3 thru_hole rect (at 0 0 145.0) (size 1.7 1.7) (drill 1) (layers *.Cu *.Mask)))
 (gr_line (start 125.000 75.000) (end 125.000 125.000) (angle 90) (layer Edge.Cuts) (width 0.15))
 (gr_line (start 175.000 75.000) (end 175.000 125.000) (angle 90) (layer Edge.Cuts) (width 0.15))
 (gr_line (start 125.000 75.000) (end 175.000 75.000) (angle 0) (layer Edge.Cuts) (width 0.15))
 (gr_line (start 125.000 125.000) (end 175.000 125.000) (angle 0) (layer Edge.Cuts) (width 0.15))
 (segment (start 131.434 108.658) (end 135.706 106.665) (width 0.2) (layer F.Cu) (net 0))
 (via (at 135.706 106.665) (size 0.6) (drill 0.4) (layers F.Cu B.Cu) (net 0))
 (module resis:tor (layer F.Cu) (at 150 100 205.0)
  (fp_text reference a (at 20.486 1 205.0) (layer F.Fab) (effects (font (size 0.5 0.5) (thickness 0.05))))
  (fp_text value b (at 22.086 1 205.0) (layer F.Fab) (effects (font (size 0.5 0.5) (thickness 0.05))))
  (pad 1 smd rect (at 20.5 0 205.0) (size 0.8 0.8) (layers F.Cu F.Paste F.Mask))
  (pad 2 smd rect (at 22.1 0 205.0) (size 0.8 0.8) (layers F.Cu F.Paste F.Mask)))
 (segment (start 129.984 109.334) (end 128.016 110.252) (width 0.2) (layer F.Cu) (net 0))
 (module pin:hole (layer F.Cu) (at 128.016 110.252)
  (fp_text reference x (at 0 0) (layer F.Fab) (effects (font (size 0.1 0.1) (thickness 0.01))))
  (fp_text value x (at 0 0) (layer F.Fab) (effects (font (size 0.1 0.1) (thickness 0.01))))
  (pad 4 thru_hole rect (at 0 0 205.0) (size 1.7 1.7) (drill 1) (layers *.Cu *.Mask)))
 (gr_line (start 125.000 75.000) (end 125.000 125.000) (angle 90) (layer Edge.Cuts) (width 0.15))
 (gr_line (start 175.000 75.000) (end 175.000 125.000) (angle 90) (layer Edge.Cuts) (width 0.15))
 (gr_line (start 125.000 75.000) (end 175.000 75.000) (angle 0) (layer Edge.Cuts) (width 0.15))
 (gr_line (start 125.000 125.000) (end 175.000 125.000) (angle 0) (layer Edge.Cuts) (width 0.15))
 (segment (start 138.250 116.781) (end 140.413 113.692) (width 0.2) (layer F.Cu) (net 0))
 (via (at 140.413 113.692) (size 0.6) (drill 0.4) (layers F.Cu B.Cu) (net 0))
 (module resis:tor (layer F.Cu) (at 150 100 235.0)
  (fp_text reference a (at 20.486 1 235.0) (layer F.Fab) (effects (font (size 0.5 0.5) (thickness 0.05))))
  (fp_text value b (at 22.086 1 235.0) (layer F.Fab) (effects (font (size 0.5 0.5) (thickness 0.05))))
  (pad 1 smd rect (at 20.5 0 235.0) (size 0.8 0.8) (layers F.Cu F.Paste F.Mask))
  (pad 2 smd rect (at 22.1 0 235.0) (size 0.8 0.8) (layers F.Cu F.Paste F.Mask)))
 (segment (start 137.332 118.092) (end 136.087 119.870) (width 0.2) (layer F.Cu) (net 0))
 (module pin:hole (layer F.Cu) (at 136.087 119.870)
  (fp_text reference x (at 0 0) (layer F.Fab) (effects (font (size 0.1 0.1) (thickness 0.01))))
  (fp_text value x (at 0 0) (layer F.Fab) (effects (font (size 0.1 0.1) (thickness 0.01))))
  (pad 5 thru_hole rect (at 0 0 235.0) (size 1.7 1.7) (drill 1) (layers *.Cu *.Mask)))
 (gr_line (start 125.000 75.000) (end 125.000 125.000) (angle 90) (layer Edge.Cuts) (width 0.15))
 (gr_line (start 175.000 75.000) (end 175.000 125.000) (angle 90) (layer Edge.Cuts) (width 0.15))
 (gr_line (start 125.000 75.000) (end 175.000 75.000) (angle 0) (layer Edge.Cuts) (width 0.15))
 (gr_line (start 125.000 125.000) (end 175.000 125.000) (angle 0) (layer Edge.Cuts) (width 0.15))
 (segment (start 158.658 118.566) (end 157.462 116.003) (width 0.2) (layer F.Cu) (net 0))
 (via (at 157.462 116.003) (size 0.6) (drill 0.4) (layers F.Cu B.Cu) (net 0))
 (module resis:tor (layer F.Cu) (at 150 100 295.0)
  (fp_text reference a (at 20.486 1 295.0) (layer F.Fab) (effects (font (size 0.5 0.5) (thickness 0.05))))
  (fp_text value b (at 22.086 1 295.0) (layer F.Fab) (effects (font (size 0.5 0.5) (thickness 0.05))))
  (pad 1 smd rect (at 20.5 0 295.0) (size 0.8 0.8) (layers F.Cu F.Paste F.Mask))
  (pad 2 smd rect (at 22.1 0 295.0) (size 0.8 0.8) (layers F.Cu F.Paste F.Mask)))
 (segment (start 159.334 120.016) (end 160.252 121.984) (width 0.2) (layer F.Cu) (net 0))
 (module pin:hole (layer F.Cu) (at 160.252 121.984)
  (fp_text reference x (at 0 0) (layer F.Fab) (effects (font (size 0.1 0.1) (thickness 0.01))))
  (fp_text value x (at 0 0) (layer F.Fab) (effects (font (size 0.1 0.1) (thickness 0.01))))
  (pad 6 thru_hole rect (at 0 0 295.0) (size 1.7 1.7) (drill 1) (layers *.Cu *.Mask)))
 (gr_line (start 125.000 75.000) (end 125.000 125.000) (angle 90) (layer Edge.Cuts) (width 0.15))
 (gr_line (start 175.000 75.000) (end 175.000 125.000) (angle 90) (layer Edge.Cuts) (width 0.15))
 (gr_line (start 125.000 75.000) (end 175.000 75.000) (angle 0) (layer Edge.Cuts) (width 0.15))
 (gr_line (start 125.000 125.000) (end 175.000 125.000) (angle 0) (layer Edge.Cuts) (width 0.15))
 (segment (start 166.781 111.750) (end 165.236 110.669) (width 0.2) (layer F.Cu) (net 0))
 (via (at 165.236 110.669) (size 0.6) (drill 0.4) (layers F.Cu B.Cu) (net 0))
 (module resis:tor (layer F.Cu) (at 150 100 325.0)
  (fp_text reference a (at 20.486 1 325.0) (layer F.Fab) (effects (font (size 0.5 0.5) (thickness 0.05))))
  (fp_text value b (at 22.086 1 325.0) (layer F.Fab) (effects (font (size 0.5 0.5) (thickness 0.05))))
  (pad 1 smd rect (at 20.5 0 325.0) (size 0.8 0.8) (layers F.Cu F.Paste F.Mask))
  (pad 2 smd rect (at 22.1 0 325.0) (size 0.8 0.8) (layers F.Cu F.Paste F.Mask)))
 (segment (start 168.092 112.668) (end 169.870 113.913) (width 0.2) (layer F.Cu) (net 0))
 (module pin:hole (layer F.Cu) (at 169.870 113.913)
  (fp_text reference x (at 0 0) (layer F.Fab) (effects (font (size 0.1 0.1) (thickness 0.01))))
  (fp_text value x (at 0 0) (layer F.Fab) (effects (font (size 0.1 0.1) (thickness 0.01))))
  (pad 7 thru_hole rect (at 0 0 325.0) (size 1.7 1.7) (drill 1) (layers *.Cu *.Mask)))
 (gr_line (start 125.000 75.000) (end 125.000 125.000) (angle 90) (layer Edge.Cuts) (width 0.15))
 (gr_line (start 175.000 75.000) (end 175.000 125.000) (angle 90) (layer Edge.Cuts) (width 0.15))
 (gr_line (start 125.000 75.000) (end 175.000 75.000) (angle 0) (layer Edge.Cuts) (width 0.15))
 (gr_line (start 125.000 125.000) (end 175.000 125.000) (angle 0) (layer Edge.Cuts) (width 0.15)))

